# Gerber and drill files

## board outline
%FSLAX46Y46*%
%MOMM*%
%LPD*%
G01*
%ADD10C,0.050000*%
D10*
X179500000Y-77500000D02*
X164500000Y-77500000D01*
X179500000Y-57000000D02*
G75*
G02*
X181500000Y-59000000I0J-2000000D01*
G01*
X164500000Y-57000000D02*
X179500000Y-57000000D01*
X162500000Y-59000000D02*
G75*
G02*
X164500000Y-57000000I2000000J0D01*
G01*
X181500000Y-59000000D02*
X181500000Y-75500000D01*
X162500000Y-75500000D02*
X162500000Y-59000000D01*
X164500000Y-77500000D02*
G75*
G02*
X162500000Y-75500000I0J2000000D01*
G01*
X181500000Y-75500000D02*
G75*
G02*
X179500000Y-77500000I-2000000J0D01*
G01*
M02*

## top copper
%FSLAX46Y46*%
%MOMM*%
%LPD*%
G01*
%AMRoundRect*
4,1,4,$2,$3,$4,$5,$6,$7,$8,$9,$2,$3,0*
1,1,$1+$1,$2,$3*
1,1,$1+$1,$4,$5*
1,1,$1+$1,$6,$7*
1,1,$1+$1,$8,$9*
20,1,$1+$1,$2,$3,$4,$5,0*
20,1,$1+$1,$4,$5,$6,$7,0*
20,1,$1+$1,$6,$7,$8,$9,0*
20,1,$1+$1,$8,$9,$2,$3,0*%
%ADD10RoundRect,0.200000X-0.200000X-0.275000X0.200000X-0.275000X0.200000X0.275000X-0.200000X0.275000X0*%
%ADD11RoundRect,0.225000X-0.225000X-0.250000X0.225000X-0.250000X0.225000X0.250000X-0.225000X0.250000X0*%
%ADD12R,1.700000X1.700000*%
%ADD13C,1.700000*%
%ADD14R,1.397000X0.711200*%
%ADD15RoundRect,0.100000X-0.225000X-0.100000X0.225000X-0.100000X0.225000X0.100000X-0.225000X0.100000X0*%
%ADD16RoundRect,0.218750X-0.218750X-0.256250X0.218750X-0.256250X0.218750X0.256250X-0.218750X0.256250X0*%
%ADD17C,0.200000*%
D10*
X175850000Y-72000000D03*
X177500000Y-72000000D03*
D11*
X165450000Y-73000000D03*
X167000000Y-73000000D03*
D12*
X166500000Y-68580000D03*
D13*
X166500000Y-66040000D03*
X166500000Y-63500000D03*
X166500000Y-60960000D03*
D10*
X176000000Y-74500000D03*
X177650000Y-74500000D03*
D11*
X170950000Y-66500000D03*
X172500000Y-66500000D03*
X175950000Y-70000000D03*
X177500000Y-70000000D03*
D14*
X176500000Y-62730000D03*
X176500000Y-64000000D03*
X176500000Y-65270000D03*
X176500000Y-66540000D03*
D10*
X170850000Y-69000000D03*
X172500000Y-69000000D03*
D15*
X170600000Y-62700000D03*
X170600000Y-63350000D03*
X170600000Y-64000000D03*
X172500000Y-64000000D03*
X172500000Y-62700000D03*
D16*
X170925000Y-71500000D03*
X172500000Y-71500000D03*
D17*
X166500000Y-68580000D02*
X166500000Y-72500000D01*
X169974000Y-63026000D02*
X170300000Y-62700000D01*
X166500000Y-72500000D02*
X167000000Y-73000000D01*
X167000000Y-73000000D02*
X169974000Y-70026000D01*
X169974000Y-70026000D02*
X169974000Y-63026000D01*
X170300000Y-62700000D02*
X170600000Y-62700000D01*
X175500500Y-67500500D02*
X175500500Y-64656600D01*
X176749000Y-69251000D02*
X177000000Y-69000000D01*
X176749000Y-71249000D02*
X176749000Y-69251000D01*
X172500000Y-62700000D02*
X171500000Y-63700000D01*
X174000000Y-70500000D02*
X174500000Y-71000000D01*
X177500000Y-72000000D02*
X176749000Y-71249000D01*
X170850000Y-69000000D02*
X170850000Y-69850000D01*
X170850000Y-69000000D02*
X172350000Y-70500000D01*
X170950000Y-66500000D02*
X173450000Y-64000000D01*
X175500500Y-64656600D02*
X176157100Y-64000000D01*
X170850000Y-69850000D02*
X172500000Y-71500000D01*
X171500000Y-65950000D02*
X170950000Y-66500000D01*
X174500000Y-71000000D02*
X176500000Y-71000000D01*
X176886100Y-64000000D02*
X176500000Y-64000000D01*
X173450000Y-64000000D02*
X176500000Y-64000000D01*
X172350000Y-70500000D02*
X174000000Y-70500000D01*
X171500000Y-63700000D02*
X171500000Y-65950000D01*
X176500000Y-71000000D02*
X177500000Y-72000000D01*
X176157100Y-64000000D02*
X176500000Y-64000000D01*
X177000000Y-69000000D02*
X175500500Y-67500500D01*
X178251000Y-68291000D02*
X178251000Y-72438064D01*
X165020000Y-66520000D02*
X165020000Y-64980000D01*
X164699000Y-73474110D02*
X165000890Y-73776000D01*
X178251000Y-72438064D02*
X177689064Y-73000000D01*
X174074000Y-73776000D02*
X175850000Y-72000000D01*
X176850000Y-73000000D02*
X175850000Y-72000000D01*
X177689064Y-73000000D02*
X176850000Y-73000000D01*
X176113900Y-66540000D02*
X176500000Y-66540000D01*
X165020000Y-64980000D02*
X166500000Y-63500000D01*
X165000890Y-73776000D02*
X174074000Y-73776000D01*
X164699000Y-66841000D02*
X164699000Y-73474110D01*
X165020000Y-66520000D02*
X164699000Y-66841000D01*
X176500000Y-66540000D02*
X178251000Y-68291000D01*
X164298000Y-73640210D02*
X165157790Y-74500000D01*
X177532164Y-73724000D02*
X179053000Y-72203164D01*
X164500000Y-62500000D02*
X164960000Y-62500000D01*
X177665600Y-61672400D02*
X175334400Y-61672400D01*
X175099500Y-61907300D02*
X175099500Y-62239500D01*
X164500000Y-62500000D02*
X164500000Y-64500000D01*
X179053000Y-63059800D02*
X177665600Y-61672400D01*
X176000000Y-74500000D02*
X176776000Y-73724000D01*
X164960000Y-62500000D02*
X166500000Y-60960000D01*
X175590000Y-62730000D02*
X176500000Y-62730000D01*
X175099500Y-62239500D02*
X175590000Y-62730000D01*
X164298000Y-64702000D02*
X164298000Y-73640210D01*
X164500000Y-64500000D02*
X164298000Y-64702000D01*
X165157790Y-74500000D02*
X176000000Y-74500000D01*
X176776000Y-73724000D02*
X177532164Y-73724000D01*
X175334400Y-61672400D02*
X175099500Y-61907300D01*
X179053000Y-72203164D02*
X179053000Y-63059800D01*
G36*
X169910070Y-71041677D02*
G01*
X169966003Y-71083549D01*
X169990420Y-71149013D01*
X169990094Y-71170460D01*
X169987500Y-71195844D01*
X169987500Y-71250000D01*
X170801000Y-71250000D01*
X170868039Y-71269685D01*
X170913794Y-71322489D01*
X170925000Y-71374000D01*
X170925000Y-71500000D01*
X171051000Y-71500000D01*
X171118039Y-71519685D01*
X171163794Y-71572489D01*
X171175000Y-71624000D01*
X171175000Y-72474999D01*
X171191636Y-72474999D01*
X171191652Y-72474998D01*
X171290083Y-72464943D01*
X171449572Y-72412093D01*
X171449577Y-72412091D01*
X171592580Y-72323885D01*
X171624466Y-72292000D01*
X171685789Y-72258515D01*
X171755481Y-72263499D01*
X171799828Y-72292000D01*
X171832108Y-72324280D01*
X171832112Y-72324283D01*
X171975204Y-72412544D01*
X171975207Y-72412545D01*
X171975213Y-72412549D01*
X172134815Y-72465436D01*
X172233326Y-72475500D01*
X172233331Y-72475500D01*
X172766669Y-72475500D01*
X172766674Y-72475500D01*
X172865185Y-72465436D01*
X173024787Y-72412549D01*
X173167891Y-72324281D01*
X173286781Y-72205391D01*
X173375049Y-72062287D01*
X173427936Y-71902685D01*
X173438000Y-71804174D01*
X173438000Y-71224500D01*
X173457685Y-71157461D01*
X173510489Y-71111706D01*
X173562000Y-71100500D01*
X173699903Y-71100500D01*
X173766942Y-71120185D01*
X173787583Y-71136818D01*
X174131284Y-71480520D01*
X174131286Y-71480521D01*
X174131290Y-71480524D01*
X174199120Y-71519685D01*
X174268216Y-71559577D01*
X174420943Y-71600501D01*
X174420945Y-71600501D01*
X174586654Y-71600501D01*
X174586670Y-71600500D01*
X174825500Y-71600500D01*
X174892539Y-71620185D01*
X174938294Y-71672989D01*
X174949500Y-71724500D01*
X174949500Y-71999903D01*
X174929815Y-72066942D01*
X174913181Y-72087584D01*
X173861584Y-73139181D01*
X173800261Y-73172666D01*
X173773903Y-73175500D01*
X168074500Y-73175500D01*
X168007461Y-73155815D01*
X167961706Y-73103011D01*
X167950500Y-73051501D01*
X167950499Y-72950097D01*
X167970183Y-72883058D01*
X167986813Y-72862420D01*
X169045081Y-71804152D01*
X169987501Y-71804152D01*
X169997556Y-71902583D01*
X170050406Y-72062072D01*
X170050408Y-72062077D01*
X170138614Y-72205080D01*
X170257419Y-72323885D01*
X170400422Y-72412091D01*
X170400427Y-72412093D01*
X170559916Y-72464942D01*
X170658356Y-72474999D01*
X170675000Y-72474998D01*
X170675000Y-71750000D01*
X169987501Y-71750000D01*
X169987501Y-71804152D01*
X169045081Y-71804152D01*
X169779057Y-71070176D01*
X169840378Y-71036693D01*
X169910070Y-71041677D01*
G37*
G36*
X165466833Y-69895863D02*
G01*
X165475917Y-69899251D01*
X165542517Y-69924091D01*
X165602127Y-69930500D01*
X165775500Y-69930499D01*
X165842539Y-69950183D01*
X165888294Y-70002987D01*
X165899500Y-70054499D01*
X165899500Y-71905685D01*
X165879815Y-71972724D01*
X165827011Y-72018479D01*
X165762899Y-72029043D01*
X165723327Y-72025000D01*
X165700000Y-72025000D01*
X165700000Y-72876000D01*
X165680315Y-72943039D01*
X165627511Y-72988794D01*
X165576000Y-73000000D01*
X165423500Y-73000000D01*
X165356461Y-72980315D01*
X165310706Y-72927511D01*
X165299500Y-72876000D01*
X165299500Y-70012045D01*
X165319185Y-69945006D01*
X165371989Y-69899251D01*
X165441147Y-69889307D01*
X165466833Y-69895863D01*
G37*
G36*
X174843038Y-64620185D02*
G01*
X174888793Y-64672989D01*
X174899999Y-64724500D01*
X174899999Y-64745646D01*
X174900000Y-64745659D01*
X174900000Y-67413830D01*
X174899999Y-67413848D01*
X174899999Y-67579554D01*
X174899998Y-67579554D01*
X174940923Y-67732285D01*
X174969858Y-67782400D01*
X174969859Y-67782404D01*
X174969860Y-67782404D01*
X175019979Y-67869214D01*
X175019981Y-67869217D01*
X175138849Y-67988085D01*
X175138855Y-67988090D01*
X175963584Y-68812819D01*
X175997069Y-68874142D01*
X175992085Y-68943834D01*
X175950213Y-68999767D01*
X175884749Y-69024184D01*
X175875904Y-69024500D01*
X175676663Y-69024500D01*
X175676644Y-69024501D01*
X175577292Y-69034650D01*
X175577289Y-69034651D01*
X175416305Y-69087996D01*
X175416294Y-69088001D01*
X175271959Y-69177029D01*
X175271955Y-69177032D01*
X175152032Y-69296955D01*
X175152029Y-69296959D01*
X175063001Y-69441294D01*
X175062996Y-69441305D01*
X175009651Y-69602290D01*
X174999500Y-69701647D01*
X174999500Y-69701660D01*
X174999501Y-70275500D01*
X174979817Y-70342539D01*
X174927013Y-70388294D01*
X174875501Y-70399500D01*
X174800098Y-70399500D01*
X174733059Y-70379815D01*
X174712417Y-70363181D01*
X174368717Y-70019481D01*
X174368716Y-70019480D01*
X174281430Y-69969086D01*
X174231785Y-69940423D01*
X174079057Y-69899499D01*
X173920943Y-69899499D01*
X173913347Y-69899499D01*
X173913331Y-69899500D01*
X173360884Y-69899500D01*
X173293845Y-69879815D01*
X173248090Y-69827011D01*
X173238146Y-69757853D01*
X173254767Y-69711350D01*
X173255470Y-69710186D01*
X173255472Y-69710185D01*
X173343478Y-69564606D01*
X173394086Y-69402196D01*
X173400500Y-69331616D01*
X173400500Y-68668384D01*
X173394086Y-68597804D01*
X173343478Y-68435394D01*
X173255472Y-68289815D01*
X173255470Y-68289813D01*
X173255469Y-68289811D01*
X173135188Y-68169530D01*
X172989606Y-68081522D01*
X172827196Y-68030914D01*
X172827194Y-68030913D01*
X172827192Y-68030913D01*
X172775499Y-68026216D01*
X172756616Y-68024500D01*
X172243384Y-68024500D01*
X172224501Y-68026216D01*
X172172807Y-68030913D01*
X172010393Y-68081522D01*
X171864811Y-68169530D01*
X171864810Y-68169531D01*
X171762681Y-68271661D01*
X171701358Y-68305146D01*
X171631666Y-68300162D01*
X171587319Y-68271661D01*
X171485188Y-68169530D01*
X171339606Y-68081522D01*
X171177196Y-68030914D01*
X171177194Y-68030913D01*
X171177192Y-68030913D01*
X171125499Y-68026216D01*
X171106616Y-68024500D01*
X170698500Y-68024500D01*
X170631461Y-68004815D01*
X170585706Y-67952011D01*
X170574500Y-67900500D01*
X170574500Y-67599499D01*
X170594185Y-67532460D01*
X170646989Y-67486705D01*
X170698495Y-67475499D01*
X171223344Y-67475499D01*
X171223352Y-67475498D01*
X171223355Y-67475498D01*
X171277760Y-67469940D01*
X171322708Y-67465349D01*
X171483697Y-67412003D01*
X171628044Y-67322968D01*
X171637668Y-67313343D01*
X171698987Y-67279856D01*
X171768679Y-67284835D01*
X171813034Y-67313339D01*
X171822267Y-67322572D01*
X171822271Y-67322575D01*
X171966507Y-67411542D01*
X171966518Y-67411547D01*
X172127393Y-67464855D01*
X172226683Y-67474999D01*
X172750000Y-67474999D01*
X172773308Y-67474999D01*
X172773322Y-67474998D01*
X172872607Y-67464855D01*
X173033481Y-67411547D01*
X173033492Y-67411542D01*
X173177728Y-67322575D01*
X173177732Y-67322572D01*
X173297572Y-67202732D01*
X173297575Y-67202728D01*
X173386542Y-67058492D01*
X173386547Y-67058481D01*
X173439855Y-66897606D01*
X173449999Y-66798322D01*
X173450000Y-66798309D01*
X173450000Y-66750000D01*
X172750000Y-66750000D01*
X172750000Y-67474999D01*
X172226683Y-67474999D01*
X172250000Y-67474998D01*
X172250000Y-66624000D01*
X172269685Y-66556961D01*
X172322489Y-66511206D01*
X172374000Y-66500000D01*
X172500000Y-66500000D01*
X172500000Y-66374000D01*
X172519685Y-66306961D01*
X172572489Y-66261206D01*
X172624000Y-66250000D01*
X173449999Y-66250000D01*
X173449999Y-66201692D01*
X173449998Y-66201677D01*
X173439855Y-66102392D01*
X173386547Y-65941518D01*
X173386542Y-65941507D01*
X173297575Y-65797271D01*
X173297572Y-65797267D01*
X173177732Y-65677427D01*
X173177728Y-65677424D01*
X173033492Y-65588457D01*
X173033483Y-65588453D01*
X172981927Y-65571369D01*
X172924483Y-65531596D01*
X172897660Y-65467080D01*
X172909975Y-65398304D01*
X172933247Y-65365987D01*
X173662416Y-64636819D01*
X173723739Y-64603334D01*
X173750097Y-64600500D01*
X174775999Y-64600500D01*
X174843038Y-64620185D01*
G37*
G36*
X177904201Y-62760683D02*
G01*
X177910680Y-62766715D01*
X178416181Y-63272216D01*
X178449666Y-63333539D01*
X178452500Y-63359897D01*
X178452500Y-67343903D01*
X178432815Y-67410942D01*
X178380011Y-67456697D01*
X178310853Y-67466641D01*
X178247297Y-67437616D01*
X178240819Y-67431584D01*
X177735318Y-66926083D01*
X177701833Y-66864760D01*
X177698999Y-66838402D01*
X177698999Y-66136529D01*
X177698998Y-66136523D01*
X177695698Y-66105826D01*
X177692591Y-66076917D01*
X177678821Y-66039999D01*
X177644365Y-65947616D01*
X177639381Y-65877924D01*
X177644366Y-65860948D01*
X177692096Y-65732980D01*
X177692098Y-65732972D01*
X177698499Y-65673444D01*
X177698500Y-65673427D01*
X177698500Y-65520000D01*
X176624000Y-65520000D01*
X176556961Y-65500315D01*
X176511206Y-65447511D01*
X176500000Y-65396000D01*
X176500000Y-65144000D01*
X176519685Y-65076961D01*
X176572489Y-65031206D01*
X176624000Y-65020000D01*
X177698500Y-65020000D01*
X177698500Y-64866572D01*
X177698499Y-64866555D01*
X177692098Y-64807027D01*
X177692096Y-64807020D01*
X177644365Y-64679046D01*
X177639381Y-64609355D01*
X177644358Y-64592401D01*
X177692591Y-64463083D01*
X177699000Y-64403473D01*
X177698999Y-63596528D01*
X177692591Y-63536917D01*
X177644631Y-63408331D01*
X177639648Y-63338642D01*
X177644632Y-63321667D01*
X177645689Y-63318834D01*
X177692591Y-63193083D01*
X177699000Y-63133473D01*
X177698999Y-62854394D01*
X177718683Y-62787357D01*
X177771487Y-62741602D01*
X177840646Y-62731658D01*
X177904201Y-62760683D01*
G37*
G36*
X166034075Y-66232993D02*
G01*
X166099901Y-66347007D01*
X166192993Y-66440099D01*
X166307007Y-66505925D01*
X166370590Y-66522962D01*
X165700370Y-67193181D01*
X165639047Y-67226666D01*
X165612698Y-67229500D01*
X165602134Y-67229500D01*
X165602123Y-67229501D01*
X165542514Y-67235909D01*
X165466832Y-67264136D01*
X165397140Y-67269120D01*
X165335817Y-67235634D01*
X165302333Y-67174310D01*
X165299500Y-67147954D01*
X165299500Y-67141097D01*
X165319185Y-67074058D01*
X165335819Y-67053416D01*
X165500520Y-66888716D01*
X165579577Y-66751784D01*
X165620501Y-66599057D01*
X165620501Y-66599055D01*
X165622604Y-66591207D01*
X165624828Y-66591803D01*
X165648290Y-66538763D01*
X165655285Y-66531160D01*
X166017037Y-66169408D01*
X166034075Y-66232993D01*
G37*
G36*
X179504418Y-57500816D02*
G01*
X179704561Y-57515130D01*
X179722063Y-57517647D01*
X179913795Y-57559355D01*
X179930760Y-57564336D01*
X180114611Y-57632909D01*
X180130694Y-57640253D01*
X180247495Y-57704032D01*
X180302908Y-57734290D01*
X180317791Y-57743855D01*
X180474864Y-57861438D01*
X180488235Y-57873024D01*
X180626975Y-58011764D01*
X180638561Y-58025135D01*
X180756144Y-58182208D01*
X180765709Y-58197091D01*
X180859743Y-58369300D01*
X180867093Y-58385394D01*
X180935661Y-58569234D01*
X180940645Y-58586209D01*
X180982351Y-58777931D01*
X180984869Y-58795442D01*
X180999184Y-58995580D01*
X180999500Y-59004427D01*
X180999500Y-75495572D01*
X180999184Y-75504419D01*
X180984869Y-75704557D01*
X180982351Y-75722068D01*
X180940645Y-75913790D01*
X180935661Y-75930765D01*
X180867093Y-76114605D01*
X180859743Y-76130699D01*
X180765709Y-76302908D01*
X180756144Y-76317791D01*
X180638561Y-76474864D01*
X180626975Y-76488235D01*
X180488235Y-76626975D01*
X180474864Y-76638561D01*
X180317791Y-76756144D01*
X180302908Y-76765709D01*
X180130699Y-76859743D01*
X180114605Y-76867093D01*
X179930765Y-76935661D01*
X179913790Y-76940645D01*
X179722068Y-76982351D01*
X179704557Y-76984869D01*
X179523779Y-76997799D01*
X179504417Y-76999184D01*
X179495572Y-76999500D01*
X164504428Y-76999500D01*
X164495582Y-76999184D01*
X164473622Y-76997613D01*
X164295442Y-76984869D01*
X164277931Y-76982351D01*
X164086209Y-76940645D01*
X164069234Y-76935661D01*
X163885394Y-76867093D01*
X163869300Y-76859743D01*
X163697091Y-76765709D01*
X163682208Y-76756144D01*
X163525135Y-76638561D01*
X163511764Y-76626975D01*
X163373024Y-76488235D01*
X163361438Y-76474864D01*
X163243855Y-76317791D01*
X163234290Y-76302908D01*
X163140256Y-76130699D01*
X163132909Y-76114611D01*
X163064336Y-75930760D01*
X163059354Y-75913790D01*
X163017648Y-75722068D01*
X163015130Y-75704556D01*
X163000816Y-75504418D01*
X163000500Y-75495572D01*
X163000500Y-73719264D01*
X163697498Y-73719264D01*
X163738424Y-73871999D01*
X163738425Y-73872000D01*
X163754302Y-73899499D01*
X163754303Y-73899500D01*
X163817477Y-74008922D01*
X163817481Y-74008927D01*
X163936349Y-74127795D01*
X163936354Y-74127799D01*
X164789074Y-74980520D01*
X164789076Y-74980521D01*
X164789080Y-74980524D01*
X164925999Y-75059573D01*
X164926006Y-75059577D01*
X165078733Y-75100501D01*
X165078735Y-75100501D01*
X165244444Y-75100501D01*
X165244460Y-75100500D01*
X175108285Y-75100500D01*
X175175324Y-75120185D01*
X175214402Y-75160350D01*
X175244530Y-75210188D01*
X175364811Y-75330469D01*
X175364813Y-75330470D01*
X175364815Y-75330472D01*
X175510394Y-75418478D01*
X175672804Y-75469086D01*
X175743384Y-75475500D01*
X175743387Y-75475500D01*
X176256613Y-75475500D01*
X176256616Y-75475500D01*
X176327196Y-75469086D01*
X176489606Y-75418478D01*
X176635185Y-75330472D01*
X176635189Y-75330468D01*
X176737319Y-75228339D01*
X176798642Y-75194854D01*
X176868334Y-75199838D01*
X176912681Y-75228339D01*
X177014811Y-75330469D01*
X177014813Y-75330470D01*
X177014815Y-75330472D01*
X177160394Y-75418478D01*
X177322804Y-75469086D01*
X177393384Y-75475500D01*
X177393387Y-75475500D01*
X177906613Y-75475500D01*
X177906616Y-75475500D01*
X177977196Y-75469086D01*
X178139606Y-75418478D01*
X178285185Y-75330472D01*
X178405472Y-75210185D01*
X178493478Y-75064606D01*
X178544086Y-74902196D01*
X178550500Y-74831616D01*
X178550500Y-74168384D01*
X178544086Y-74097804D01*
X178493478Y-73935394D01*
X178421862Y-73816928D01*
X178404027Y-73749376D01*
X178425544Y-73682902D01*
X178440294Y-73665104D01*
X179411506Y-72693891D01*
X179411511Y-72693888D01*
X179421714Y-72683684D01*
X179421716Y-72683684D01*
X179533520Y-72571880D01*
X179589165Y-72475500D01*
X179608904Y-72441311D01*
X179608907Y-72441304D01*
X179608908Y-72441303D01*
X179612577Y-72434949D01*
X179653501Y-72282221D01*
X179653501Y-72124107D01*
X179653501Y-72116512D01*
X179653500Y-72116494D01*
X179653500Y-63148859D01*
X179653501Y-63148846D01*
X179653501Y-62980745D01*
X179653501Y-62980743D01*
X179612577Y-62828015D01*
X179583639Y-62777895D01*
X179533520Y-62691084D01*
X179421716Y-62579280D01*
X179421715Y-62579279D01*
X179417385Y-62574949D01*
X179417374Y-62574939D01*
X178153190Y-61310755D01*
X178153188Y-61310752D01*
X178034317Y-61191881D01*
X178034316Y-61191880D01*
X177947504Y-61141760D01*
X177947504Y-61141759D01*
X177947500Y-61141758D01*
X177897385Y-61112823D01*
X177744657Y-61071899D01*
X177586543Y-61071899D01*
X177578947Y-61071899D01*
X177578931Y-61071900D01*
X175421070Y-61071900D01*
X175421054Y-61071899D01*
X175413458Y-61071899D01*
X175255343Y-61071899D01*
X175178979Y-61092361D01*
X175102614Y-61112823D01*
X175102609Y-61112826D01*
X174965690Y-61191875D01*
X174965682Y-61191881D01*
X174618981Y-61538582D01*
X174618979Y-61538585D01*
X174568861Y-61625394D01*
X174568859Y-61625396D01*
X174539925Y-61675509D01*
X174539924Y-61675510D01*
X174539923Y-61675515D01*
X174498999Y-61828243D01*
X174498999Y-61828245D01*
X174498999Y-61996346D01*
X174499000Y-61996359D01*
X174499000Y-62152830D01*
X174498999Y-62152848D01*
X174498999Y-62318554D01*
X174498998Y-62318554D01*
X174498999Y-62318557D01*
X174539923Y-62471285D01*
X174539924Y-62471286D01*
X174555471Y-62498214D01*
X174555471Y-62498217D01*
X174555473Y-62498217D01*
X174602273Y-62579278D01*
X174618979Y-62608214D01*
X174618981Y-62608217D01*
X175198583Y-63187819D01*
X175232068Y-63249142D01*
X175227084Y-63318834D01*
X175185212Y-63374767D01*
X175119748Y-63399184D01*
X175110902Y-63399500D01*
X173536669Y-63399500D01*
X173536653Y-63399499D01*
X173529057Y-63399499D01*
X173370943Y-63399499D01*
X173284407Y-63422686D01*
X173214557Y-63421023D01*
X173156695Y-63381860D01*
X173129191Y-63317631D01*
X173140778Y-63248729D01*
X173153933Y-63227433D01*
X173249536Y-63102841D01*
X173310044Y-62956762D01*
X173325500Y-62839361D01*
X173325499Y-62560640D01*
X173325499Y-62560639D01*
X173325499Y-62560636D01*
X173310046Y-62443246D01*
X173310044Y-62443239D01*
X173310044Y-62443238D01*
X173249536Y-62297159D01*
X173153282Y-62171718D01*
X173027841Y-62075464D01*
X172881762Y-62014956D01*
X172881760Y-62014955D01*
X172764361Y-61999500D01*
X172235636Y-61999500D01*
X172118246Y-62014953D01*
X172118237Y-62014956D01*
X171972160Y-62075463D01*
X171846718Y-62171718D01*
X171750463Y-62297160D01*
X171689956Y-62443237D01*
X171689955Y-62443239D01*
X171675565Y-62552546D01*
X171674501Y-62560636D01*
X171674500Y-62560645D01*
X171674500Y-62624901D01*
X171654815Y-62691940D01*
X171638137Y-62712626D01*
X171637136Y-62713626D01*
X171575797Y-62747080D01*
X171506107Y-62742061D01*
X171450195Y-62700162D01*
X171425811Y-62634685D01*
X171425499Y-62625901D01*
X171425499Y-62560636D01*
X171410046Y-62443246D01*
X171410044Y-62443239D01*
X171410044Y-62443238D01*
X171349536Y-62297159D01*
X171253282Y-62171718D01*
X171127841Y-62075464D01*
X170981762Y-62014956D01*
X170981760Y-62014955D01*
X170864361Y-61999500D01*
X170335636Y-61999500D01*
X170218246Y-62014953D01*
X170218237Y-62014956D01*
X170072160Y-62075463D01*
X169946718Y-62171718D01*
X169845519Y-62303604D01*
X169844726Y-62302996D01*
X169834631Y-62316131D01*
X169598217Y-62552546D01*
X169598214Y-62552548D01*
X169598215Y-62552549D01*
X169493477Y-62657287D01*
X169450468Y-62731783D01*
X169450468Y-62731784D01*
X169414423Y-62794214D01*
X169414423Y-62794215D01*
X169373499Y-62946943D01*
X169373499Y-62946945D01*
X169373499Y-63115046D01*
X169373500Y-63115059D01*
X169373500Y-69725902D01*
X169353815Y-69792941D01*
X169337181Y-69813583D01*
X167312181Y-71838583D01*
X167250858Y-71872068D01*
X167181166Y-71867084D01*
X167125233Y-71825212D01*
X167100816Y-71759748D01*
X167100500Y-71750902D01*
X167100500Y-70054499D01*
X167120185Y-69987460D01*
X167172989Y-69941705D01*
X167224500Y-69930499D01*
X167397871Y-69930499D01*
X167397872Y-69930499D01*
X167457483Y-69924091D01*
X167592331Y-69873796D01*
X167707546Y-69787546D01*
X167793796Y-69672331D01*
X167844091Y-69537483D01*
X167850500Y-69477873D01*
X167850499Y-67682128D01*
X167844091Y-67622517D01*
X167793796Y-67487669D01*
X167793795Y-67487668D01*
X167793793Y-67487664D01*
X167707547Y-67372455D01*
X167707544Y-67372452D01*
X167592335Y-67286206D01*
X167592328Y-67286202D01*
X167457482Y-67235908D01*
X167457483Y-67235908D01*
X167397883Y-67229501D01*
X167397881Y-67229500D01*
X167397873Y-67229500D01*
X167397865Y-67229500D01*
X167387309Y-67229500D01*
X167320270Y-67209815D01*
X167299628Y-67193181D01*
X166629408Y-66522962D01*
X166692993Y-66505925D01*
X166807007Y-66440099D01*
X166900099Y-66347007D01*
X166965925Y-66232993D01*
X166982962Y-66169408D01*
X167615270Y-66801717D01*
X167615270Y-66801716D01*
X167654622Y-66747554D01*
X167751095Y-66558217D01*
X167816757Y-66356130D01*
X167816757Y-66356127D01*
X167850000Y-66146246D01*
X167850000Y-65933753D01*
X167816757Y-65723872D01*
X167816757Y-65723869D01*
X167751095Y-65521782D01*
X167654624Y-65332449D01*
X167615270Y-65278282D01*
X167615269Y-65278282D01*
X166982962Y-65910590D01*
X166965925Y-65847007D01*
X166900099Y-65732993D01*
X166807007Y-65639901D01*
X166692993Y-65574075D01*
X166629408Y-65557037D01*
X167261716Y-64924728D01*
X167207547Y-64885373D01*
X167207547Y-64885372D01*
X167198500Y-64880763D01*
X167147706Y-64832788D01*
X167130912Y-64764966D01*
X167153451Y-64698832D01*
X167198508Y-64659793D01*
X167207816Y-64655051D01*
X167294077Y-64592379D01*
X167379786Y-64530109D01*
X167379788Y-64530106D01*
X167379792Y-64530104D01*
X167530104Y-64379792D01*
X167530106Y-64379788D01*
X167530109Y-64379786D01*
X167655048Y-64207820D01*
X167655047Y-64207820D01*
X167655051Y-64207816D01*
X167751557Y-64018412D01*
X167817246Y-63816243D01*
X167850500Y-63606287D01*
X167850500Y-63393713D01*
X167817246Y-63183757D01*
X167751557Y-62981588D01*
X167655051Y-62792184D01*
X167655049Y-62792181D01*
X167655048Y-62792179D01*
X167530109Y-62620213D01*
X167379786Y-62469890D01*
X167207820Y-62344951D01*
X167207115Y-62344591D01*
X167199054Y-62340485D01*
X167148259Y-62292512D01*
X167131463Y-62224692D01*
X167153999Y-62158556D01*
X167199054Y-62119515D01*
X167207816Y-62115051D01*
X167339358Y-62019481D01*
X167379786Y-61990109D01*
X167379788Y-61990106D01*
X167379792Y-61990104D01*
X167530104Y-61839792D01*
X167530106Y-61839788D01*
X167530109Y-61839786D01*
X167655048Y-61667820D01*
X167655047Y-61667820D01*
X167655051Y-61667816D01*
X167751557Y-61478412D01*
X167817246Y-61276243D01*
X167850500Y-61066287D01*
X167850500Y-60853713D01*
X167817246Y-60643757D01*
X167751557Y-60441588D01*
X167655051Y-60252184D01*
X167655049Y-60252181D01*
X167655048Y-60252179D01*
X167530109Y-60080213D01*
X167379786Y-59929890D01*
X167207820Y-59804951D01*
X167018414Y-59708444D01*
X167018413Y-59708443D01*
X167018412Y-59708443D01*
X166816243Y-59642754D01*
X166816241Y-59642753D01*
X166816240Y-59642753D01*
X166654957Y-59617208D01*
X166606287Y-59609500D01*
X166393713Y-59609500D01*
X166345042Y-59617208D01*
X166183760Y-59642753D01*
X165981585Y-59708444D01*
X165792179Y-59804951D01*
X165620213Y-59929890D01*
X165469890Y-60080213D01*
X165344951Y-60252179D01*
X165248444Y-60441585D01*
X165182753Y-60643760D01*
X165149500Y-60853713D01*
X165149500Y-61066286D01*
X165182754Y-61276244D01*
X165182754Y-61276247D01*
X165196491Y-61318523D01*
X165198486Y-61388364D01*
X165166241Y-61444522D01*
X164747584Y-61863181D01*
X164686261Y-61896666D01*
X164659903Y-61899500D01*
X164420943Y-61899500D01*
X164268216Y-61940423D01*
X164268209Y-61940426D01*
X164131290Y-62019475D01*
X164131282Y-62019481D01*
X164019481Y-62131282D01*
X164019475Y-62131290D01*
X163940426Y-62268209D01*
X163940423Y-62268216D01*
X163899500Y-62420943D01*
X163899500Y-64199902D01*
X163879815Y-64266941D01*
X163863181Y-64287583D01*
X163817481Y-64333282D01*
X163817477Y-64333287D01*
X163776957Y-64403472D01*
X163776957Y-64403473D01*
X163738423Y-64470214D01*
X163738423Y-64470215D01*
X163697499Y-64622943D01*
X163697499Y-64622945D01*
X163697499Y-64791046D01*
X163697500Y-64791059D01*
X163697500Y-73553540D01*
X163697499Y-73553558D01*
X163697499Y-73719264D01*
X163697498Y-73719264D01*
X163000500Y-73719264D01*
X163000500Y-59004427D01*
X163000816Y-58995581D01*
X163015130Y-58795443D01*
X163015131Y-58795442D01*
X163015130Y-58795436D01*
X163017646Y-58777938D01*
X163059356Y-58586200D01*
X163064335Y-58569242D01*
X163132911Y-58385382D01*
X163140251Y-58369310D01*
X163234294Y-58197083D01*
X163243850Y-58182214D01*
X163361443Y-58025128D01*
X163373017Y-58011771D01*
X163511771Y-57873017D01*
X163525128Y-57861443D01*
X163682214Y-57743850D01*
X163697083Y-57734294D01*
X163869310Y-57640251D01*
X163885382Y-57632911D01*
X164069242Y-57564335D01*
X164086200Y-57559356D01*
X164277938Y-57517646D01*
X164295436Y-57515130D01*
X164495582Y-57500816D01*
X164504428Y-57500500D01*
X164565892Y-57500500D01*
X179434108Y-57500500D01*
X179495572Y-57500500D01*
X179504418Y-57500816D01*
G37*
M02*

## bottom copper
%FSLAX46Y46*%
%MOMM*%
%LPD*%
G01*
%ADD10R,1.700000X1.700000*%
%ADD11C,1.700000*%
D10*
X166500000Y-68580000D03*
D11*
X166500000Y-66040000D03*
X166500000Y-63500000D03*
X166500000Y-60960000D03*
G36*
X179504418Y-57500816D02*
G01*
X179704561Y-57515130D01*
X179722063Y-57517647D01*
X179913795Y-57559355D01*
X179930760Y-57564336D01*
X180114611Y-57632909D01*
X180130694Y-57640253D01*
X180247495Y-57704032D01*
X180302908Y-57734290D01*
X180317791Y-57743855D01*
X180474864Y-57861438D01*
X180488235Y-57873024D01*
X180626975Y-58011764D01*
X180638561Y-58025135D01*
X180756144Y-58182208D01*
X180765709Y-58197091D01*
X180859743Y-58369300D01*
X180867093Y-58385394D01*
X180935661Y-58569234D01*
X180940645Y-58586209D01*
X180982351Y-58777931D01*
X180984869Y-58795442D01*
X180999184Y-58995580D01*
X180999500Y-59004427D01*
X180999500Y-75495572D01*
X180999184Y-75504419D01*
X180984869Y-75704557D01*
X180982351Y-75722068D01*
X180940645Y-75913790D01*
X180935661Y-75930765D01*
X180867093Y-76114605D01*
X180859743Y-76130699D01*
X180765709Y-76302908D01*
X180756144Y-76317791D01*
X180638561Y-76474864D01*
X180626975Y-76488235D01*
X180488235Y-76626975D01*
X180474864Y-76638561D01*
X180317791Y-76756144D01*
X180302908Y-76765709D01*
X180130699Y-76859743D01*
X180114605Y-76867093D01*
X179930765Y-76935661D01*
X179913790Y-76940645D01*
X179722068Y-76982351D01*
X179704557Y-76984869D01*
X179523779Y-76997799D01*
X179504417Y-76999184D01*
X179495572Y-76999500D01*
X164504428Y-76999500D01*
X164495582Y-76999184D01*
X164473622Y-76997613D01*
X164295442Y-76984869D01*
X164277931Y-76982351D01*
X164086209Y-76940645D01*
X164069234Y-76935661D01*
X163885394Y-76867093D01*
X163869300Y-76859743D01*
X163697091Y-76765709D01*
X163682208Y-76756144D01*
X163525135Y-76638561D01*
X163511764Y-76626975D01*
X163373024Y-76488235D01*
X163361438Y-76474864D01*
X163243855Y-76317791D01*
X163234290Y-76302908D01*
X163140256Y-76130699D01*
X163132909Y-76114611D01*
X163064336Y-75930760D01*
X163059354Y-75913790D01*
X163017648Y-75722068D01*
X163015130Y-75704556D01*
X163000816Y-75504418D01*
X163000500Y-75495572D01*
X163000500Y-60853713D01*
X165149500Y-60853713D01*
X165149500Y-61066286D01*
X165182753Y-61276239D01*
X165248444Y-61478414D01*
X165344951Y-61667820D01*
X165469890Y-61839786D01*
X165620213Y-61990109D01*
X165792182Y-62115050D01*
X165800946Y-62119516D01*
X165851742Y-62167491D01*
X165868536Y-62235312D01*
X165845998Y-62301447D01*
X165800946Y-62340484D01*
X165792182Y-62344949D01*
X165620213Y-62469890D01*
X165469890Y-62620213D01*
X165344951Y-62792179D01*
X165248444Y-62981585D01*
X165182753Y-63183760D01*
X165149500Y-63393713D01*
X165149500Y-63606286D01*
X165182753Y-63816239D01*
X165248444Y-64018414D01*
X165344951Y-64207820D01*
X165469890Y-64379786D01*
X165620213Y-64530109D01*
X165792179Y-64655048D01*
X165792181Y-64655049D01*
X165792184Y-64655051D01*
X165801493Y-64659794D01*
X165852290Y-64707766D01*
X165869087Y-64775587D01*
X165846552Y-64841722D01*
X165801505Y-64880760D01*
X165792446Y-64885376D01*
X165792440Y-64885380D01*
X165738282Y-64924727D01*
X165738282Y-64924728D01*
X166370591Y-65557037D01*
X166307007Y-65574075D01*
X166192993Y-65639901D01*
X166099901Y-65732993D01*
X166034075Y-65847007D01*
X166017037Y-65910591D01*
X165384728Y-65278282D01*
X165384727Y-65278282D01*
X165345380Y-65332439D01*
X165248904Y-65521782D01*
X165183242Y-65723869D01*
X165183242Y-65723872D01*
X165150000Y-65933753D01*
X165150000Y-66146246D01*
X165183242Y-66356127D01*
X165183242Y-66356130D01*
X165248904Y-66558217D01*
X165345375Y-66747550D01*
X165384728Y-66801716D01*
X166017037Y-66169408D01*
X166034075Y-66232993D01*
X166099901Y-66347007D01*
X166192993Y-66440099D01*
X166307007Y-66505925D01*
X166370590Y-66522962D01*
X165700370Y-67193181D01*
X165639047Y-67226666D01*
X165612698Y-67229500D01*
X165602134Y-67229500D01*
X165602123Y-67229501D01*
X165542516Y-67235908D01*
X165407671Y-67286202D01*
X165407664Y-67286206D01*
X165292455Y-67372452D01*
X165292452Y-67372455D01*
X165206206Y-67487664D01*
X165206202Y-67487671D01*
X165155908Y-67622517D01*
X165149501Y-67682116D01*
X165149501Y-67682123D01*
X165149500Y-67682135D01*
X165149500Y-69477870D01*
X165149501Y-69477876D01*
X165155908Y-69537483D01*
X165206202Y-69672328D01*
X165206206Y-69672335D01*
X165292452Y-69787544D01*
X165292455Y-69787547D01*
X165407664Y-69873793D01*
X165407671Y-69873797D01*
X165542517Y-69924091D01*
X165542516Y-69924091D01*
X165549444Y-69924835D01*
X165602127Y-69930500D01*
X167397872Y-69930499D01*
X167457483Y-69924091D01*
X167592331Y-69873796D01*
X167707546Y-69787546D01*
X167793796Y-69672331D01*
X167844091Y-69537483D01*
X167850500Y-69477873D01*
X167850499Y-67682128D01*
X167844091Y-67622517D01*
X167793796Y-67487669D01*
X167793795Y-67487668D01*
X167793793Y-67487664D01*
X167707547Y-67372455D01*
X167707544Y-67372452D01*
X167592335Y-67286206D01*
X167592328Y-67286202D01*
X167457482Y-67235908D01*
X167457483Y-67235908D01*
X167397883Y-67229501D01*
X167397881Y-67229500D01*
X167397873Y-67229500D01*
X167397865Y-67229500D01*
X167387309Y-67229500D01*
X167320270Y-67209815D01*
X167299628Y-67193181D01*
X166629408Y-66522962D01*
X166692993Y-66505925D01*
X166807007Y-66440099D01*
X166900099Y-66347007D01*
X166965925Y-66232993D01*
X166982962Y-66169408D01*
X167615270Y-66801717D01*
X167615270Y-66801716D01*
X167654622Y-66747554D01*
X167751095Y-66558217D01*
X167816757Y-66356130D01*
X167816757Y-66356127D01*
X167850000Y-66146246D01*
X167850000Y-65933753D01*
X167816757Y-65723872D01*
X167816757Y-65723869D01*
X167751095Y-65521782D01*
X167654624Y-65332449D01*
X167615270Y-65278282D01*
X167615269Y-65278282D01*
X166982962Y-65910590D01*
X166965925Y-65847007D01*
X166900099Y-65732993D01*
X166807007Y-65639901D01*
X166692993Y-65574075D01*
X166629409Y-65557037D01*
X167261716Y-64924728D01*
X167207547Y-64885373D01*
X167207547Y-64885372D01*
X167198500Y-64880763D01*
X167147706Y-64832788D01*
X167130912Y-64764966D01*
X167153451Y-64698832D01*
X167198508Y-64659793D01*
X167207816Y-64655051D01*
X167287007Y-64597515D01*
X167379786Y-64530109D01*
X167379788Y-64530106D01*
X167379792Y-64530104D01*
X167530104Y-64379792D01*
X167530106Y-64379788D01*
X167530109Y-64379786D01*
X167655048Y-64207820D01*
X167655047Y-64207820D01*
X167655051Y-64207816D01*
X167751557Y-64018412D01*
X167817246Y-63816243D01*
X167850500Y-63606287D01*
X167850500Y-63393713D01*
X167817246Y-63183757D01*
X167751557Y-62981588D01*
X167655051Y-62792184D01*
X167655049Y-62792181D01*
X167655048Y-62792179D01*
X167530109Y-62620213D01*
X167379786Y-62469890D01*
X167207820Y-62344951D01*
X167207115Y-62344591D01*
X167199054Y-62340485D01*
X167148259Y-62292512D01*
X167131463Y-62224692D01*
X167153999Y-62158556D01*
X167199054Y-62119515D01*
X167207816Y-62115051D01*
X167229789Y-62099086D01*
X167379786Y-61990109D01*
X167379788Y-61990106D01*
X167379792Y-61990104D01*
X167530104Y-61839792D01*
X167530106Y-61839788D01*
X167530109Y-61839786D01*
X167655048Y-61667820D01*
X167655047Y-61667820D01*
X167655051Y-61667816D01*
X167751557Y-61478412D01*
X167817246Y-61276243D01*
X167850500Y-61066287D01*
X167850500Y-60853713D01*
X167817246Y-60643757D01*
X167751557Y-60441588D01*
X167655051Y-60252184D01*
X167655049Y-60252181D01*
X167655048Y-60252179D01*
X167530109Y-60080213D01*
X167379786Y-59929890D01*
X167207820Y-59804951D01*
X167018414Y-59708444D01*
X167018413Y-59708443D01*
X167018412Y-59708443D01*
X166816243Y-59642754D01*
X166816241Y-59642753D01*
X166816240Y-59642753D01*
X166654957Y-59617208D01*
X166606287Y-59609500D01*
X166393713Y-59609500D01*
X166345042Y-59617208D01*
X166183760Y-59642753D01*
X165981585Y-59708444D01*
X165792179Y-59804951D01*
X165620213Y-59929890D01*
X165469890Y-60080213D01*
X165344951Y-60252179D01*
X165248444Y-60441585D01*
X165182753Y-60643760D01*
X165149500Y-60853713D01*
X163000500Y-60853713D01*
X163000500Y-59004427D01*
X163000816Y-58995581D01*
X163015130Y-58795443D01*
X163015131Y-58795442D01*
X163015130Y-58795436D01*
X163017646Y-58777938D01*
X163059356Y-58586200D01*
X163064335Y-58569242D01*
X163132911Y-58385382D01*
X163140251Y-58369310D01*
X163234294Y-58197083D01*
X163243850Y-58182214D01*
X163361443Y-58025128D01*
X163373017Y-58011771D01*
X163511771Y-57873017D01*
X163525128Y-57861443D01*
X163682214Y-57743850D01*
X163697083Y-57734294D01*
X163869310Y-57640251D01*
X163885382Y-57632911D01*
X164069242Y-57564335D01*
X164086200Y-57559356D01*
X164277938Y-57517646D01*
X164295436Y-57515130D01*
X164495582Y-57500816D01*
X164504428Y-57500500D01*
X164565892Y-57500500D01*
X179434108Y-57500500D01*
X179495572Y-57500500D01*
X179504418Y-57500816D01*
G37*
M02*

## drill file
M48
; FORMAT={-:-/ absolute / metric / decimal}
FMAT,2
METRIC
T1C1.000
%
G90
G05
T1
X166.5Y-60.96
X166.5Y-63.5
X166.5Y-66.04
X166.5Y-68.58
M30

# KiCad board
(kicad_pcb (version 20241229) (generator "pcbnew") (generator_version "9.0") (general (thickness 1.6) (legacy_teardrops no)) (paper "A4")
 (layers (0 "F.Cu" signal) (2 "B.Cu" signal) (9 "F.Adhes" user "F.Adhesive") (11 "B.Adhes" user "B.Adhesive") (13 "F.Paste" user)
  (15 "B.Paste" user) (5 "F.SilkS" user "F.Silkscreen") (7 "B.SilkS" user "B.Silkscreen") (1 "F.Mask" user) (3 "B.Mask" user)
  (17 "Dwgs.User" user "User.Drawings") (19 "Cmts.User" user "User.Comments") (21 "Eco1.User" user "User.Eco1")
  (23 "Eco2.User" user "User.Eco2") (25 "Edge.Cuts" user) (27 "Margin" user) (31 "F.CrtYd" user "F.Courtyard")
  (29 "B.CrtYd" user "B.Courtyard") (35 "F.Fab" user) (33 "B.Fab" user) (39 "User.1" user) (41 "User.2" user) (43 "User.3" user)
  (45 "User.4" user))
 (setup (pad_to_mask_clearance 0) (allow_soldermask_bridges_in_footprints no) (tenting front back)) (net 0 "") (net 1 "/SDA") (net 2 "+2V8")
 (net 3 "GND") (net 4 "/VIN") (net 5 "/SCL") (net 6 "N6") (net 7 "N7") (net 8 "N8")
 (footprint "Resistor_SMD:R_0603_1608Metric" (layer "F.Cu") (at 176.675 72)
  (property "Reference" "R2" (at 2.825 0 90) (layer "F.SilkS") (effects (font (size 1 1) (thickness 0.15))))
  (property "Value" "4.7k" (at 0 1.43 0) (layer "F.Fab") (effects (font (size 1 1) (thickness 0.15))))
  (pad "1" smd roundrect (at -0.825 0) (size 0.8 0.95) (layers "F.Cu" "F.Mask" "F.Paste") (roundrect_rratio 0.25) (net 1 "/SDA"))
  (pad "2" smd roundrect (at 0.825 0) (size 0.8 0.95) (layers "F.Cu" "F.Mask" "F.Paste") (roundrect_rratio 0.25) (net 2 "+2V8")))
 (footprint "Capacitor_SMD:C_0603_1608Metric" (layer "F.Cu") (at 166.225 73)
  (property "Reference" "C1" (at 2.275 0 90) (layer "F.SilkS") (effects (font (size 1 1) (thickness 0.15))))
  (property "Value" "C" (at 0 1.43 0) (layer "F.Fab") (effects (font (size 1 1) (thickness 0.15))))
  (pad "1" smd roundrect (at -0.775 0) (size 0.9 0.95) (layers "F.Cu" "F.Mask" "F.Paste") (roundrect_rratio 0.25) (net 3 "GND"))
  (pad "2" smd roundrect (at 0.775 0) (size 0.9 0.95) (layers "F.Cu" "F.Mask" "F.Paste") (roundrect_rratio 0.25) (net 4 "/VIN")))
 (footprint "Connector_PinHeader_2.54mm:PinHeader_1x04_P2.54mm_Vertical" (layer "F.Cu") (at 166.5 68.58 180)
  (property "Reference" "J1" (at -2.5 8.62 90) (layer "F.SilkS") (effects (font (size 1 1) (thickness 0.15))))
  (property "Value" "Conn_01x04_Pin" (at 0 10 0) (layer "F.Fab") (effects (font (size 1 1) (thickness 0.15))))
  (pad "1" thru_hole rect (at 0 0 180) (size 1.7 1.7) (drill 1) (layers "*.Cu" "*.Mask") (remove_unused_layers no) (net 4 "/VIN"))
  (pad "2" thru_hole circle (at 0 2.54 180) (size 1.7 1.7) (drill 1) (layers "*.Cu" "*.Mask") (remove_unused_layers no) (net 3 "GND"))
  (pad "3" thru_hole circle (at 0 5.08 180) (size 1.7 1.7) (drill 1) (layers "*.Cu" "*.Mask") (remove_unused_layers no) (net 1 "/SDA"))
  (pad "4" thru_hole circle (at 0 7.62 180) (size 1.7 1.7) (drill 1) (layers "*.Cu" "*.Mask") (remove_unused_layers no) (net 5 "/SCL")))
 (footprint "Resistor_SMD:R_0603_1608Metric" (layer "F.Cu") (at 176.825 74.5)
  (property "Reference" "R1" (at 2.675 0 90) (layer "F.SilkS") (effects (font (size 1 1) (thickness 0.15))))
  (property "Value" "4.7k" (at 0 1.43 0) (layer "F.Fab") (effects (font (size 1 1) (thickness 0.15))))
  (pad "1" smd roundrect (at -0.825 0) (size 0.8 0.95) (layers "F.Cu" "F.Mask" "F.Paste") (roundrect_rratio 0.25) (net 5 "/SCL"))
  (pad "2" smd roundrect (at 0.825 0) (size 0.8 0.95) (layers "F.Cu" "F.Mask" "F.Paste") (roundrect_rratio 0.25) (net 2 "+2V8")))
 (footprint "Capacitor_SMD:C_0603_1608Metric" (layer "F.Cu") (at 171.725 66.5)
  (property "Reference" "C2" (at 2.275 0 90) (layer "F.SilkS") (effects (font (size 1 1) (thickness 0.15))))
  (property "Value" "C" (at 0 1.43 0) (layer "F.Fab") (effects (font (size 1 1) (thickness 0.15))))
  (pad "1" smd roundrect (at -0.775 0) (size 0.9 0.95) (layers "F.Cu" "F.Mask" "F.Paste") (roundrect_rratio 0.25) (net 2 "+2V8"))
  (pad "2" smd roundrect (at 0.775 0) (size 0.9 0.95) (layers "F.Cu" "F.Mask" "F.Paste") (roundrect_rratio 0.25) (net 3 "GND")))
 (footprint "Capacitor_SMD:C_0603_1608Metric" (layer "F.Cu") (at 176.725 70)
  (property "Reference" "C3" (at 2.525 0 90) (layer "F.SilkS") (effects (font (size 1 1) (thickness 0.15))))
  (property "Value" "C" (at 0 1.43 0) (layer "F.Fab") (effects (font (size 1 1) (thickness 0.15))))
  (pad "1" smd roundrect (at -0.775 0) (size 0.9 0.95) (layers "F.Cu" "F.Mask" "F.Paste") (roundrect_rratio 0.25) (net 2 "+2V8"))
  (pad "2" smd roundrect (at 0.775 0) (size 0.9 0.95) (layers "F.Cu" "F.Mask" "F.Paste") (roundrect_rratio 0.25) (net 3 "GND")))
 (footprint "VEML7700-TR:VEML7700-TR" (layer "F.Cu") (at 177.4752 64.635 -90)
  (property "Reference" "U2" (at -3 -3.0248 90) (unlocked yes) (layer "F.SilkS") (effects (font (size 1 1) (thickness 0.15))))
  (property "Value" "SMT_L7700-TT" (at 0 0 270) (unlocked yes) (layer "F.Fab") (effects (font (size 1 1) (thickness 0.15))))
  (pad "1" smd rect (at -1.905 0.9752 270) (size 0.7112 1.397) (layers "F.Cu" "F.Mask" "F.Paste") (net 5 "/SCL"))
  (pad "2" smd rect (at -0.635 0.9752 270) (size 0.7112 1.397) (layers "F.Cu" "F.Mask" "F.Paste") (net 2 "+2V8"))
  (pad "3" smd rect (at 0.635 0.9752 270) (size 0.7112 1.397) (layers "F.Cu" "F.Mask" "F.Paste") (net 3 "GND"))
  (pad "4" smd rect (at 1.905 0.9752 270) (size 0.7112 1.397) (layers "F.Cu" "F.Mask" "F.Paste") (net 1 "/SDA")))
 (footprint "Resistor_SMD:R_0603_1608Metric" (layer "F.Cu") (at 171.675 69)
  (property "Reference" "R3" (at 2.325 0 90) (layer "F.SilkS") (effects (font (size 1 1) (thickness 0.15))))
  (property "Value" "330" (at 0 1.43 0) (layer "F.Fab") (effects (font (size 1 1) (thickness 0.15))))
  (pad "1" smd roundrect (at -0.825 0) (size 0.8 0.95) (layers "F.Cu" "F.Mask" "F.Paste") (roundrect_rratio 0.25) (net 2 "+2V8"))
  (pad "2" smd roundrect (at 0.825 0) (size 0.8 0.95) (layers "F.Cu" "F.Mask" "F.Paste") (roundrect_rratio 0.25) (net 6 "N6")))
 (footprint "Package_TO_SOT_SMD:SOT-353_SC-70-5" (layer "F.Cu") (at 171.55 63.35)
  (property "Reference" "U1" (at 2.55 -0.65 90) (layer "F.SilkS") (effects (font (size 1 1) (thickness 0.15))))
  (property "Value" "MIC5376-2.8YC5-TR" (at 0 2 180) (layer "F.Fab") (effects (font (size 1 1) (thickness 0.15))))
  (pad "1" smd roundrect (at -0.95 -0.65) (size 0.65 0.4) (layers "F.Cu" "F.Mask" "F.Paste") (roundrect_rratio 0.25) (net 4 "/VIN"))
  (pad "2" smd roundrect (at -0.95 0) (size 0.65 0.4) (layers "F.Cu" "F.Mask" "F.Paste") (roundrect_rratio 0.25) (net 3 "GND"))
  (pad "3" smd roundrect (at -0.95 0.65) (size 0.65 0.4) (layers "F.Cu" "F.Mask" "F.Paste") (roundrect_rratio 0.25) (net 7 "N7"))
  (pad "4" smd roundrect (at 0.95 0.65) (size 0.65 0.4) (layers "F.Cu" "F.Mask" "F.Paste") (roundrect_rratio 0.25) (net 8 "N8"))
  (pad "5" smd roundrect (at 0.95 -0.65) (size 0.65 0.4) (layers "F.Cu" "F.Mask" "F.Paste") (roundrect_rratio 0.25) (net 2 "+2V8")))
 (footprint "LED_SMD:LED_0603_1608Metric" (layer "F.Cu") (at 171.7125 71.5)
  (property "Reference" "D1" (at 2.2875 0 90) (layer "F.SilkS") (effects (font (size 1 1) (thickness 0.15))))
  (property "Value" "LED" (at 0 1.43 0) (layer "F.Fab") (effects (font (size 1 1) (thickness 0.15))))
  (pad "1" smd roundrect (at -0.7875 0) (size 0.875 0.95) (layers "F.Cu" "F.Mask" "F.Paste") (roundrect_rratio 0.25) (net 3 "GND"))
  (pad "2" smd roundrect (at 0.7875 0) (size 0.875 0.95) (layers "F.Cu" "F.Mask" "F.Paste") (roundrect_rratio 0.25) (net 2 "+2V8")))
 (gr_line (start 179.5 77.5) (end 164.5 77.5) (stroke (width 0.05) (type default)) (layer "Edge.Cuts"))
 (gr_arc (start 179.5 57) (mid 180.914214 57.585786) (end 181.5 59) (stroke (width 0.05) (type default)) (layer "Edge.Cuts"))
 (gr_line (start 164.5 57) (end 179.5 57) (stroke (width 0.05) (type default)) (layer "Edge.Cuts"))
 (gr_arc (start 162.5 59) (mid 163.085786 57.585786) (end 164.5 57) (stroke (width 0.05) (type default)) (layer "Edge.Cuts"))
 (gr_line (start 181.5 59) (end 181.5 75.5) (stroke (width 0.05) (type default)) (layer "Edge.Cuts"))
 (gr_line (start 162.5 75.5) (end 162.5 59) (stroke (width 0.05) (type default)) (layer "Edge.Cuts"))
 (gr_arc (start 164.5 77.5) (mid 163.085786 76.914214) (end 162.5 75.5) (stroke (width 0.05) (type default)) (layer "Edge.Cuts"))
 (gr_arc (start 181.5 75.5) (mid 180.914214 76.914214) (end 179.5 77.5) (stroke (width 0.05) (type default)) (layer "Edge.Cuts"))
 (segment (start 166.5 68.58) (end 166.5 72.5) (width 0.2) (layer "F.Cu") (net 4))
 (segment (start 169.974 63.026) (end 170.3 62.7) (width 0.2) (layer "F.Cu") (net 4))
 (segment (start 166.5 72.5) (end 167 73) (width 0.2) (layer "F.Cu") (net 4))
 (segment (start 167 73) (end 169.974 70.026) (width 0.2) (layer "F.Cu") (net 4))
 (segment (start 169.974 70.026) (end 169.974 63.026) (width 0.2) (layer "F.Cu") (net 4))
 (segment (start 170.3 62.7) (end 170.6 62.7) (width 0.2) (layer "F.Cu") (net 4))
 (segment (start 175.5005 67.5005) (end 175.5005 64.6566) (width 0.2) (layer "F.Cu") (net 2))
 (segment (start 176.749 69.251) (end 177 69) (width 0.2) (layer "F.Cu") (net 2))
 (segment (start 176.749 71.249) (end 176.749 69.251) (width 0.2) (layer "F.Cu") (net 2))
 (segment (start 172.5 62.7) (end 171.5 63.7) (width 0.2) (layer "F.Cu") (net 2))
 (segment (start 174 70.5) (end 174.5 71) (width 0.2) (layer "F.Cu") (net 2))
 (segment (start 177.5 72) (end 176.749 71.249) (width 0.2) (layer "F.Cu") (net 2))
 (segment (start 170.85 69) (end 170.85 69.85) (width 0.2) (layer "F.Cu") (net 2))
 (segment (start 170.85 69) (end 172.35 70.5) (width 0.2) (layer "F.Cu") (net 2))
 (segment (start 170.95 66.5) (end 173.45 64) (width 0.2) (layer "F.Cu") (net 2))
 (segment (start 175.5005 64.6566) (end 176.1571 64) (width 0.2) (layer "F.Cu") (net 2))
 (segment (start 170.85 69.85) (end 172.5 71.5) (width 0.2) (layer "F.Cu") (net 2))
 (segment (start 171.5 65.95) (end 170.95 66.5) (width 0.2) (layer "F.Cu") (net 2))
 (segment (start 174.5 71) (end 176.5 71) (width 0.2) (layer "F.Cu") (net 2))
 (segment (start 176.8861 64) (end 176.5 64) (width 0.2) (layer "F.Cu") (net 2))
 (segment (start 173.45 64) (end 176.5 64) (width 0.2) (layer "F.Cu") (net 2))
 (segment (start 172.35 70.5) (end 174 70.5) (width 0.2) (layer "F.Cu") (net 2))
 (segment (start 171.5 63.7) (end 171.5 65.95) (width 0.2) (layer "F.Cu") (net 2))
 (segment (start 176.5 71) (end 177.5 72) (width 0.2) (layer "F.Cu") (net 2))
 (segment (start 176.1571 64) (end 176.5 64) (width 0.2) (layer "F.Cu") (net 2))
 (segment (start 177 69) (end 175.5005 67.5005) (width 0.2) (layer "F.Cu") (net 2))
 (segment (start 178.251 68.291) (end 178.251 72.438064) (width 0.2) (layer "F.Cu") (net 1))
 (segment (start 165.02 66.52) (end 165.02 64.98) (width 0.2) (layer "F.Cu") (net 1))
 (segment (start 164.699 73.47411) (end 165.00089 73.776) (width 0.2) (layer "F.Cu") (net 1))
 (segment (start 178.251 72.438064) (end 177.689064 73) (width 0.2) (layer "F.Cu") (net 1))
 (segment (start 174.074 73.776) (end 175.85 72) (width 0.2) (layer "F.Cu") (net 1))
 (segment (start 176.85 73) (end 175.85 72) (width 0.2) (layer "F.Cu") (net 1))
 (segment (start 177.689064 73) (end 176.85 73) (width 0.2) (layer "F.Cu") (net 1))
 (segment (start 176.1139 66.54) (end 176.5 66.54) (width 0.2) (layer "F.Cu") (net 1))
 (segment (start 165.02 64.98) (end 166.5 63.5) (width 0.2) (layer "F.Cu") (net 1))
 (segment (start 165.00089 73.776) (end 174.074 73.776) (width 0.2) (layer "F.Cu") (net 1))
 (segment (start 164.699 66.841) (end 164.699 73.47411) (width 0.2) (layer "F.Cu") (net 1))
 (segment (start 165.02 66.52) (end 164.699 66.841) (width 0.2) (layer "F.Cu") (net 1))
 (segment (start 176.5 66.54) (end 178.251 68.291) (width 0.2) (layer "F.Cu") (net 1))
 (segment (start 164.298 73.64021) (end 165.15779 74.5) (width 0.2) (layer "F.Cu") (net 5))
 (segment (start 177.532164 73.724) (end 179.053 72.203164) (width 0.2) (layer "F.Cu") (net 5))
 (segment (start 164.5 62.5) (end 164.96 62.5) (width 0.2) (layer "F.Cu") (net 5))
 (segment (start 177.6656 61.6724) (end 175.3344 61.6724) (width 0.2) (layer "F.Cu") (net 5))
 (segment (start 175.0995 61.9073) (end 175.0995 62.2395) (width 0.2) (layer "F.Cu") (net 5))
 (segment (start 164.5 62.5) (end 164.5 64.5) (width 0.2) (layer "F.Cu") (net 5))
 (segment (start 179.053 63.0598) (end 177.6656 61.6724) (width 0.2) (layer "F.Cu") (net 5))
 (segment (start 176 74.5) (end 176.776 73.724) (width 0.2) (layer "F.Cu") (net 5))
 (segment (start 164.96 62.5) (end 166.5 60.96) (width 0.2) (layer "F.Cu") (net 5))
 (segment (start 175.59 62.73) (end 176.5 62.73) (width 0.2) (layer "F.Cu") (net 5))
 (segment (start 175.0995 62.2395) (end 175.59 62.73) (width 0.2) (layer "F.Cu") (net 5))
 (segment (start 164.298 64.702) (end 164.298 73.64021) (width 0.2) (layer "F.Cu") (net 5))
 (segment (start 164.5 64.5) (end 164.298 64.702) (width 0.2) (layer "F.Cu") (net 5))
 (segment (start 165.15779 74.5) (end 176 74.5) (width 0.2) (layer "F.Cu") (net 5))
 (segment (start 176.776 73.724) (end 177.532164 73.724) (width 0.2) (layer "F.Cu") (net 5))
 (segment (start 175.3344 61.6724) (end 175.0995 61.9073) (width 0.2) (layer "F.Cu") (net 5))
 (segment (start 179.053 72.203164) (end 179.053 63.0598) (width 0.2) (layer "F.Cu") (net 5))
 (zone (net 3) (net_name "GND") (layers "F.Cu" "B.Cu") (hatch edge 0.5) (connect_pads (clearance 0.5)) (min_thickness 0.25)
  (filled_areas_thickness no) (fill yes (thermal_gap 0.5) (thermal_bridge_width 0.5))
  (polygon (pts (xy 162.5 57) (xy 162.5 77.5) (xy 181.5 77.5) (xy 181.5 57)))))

